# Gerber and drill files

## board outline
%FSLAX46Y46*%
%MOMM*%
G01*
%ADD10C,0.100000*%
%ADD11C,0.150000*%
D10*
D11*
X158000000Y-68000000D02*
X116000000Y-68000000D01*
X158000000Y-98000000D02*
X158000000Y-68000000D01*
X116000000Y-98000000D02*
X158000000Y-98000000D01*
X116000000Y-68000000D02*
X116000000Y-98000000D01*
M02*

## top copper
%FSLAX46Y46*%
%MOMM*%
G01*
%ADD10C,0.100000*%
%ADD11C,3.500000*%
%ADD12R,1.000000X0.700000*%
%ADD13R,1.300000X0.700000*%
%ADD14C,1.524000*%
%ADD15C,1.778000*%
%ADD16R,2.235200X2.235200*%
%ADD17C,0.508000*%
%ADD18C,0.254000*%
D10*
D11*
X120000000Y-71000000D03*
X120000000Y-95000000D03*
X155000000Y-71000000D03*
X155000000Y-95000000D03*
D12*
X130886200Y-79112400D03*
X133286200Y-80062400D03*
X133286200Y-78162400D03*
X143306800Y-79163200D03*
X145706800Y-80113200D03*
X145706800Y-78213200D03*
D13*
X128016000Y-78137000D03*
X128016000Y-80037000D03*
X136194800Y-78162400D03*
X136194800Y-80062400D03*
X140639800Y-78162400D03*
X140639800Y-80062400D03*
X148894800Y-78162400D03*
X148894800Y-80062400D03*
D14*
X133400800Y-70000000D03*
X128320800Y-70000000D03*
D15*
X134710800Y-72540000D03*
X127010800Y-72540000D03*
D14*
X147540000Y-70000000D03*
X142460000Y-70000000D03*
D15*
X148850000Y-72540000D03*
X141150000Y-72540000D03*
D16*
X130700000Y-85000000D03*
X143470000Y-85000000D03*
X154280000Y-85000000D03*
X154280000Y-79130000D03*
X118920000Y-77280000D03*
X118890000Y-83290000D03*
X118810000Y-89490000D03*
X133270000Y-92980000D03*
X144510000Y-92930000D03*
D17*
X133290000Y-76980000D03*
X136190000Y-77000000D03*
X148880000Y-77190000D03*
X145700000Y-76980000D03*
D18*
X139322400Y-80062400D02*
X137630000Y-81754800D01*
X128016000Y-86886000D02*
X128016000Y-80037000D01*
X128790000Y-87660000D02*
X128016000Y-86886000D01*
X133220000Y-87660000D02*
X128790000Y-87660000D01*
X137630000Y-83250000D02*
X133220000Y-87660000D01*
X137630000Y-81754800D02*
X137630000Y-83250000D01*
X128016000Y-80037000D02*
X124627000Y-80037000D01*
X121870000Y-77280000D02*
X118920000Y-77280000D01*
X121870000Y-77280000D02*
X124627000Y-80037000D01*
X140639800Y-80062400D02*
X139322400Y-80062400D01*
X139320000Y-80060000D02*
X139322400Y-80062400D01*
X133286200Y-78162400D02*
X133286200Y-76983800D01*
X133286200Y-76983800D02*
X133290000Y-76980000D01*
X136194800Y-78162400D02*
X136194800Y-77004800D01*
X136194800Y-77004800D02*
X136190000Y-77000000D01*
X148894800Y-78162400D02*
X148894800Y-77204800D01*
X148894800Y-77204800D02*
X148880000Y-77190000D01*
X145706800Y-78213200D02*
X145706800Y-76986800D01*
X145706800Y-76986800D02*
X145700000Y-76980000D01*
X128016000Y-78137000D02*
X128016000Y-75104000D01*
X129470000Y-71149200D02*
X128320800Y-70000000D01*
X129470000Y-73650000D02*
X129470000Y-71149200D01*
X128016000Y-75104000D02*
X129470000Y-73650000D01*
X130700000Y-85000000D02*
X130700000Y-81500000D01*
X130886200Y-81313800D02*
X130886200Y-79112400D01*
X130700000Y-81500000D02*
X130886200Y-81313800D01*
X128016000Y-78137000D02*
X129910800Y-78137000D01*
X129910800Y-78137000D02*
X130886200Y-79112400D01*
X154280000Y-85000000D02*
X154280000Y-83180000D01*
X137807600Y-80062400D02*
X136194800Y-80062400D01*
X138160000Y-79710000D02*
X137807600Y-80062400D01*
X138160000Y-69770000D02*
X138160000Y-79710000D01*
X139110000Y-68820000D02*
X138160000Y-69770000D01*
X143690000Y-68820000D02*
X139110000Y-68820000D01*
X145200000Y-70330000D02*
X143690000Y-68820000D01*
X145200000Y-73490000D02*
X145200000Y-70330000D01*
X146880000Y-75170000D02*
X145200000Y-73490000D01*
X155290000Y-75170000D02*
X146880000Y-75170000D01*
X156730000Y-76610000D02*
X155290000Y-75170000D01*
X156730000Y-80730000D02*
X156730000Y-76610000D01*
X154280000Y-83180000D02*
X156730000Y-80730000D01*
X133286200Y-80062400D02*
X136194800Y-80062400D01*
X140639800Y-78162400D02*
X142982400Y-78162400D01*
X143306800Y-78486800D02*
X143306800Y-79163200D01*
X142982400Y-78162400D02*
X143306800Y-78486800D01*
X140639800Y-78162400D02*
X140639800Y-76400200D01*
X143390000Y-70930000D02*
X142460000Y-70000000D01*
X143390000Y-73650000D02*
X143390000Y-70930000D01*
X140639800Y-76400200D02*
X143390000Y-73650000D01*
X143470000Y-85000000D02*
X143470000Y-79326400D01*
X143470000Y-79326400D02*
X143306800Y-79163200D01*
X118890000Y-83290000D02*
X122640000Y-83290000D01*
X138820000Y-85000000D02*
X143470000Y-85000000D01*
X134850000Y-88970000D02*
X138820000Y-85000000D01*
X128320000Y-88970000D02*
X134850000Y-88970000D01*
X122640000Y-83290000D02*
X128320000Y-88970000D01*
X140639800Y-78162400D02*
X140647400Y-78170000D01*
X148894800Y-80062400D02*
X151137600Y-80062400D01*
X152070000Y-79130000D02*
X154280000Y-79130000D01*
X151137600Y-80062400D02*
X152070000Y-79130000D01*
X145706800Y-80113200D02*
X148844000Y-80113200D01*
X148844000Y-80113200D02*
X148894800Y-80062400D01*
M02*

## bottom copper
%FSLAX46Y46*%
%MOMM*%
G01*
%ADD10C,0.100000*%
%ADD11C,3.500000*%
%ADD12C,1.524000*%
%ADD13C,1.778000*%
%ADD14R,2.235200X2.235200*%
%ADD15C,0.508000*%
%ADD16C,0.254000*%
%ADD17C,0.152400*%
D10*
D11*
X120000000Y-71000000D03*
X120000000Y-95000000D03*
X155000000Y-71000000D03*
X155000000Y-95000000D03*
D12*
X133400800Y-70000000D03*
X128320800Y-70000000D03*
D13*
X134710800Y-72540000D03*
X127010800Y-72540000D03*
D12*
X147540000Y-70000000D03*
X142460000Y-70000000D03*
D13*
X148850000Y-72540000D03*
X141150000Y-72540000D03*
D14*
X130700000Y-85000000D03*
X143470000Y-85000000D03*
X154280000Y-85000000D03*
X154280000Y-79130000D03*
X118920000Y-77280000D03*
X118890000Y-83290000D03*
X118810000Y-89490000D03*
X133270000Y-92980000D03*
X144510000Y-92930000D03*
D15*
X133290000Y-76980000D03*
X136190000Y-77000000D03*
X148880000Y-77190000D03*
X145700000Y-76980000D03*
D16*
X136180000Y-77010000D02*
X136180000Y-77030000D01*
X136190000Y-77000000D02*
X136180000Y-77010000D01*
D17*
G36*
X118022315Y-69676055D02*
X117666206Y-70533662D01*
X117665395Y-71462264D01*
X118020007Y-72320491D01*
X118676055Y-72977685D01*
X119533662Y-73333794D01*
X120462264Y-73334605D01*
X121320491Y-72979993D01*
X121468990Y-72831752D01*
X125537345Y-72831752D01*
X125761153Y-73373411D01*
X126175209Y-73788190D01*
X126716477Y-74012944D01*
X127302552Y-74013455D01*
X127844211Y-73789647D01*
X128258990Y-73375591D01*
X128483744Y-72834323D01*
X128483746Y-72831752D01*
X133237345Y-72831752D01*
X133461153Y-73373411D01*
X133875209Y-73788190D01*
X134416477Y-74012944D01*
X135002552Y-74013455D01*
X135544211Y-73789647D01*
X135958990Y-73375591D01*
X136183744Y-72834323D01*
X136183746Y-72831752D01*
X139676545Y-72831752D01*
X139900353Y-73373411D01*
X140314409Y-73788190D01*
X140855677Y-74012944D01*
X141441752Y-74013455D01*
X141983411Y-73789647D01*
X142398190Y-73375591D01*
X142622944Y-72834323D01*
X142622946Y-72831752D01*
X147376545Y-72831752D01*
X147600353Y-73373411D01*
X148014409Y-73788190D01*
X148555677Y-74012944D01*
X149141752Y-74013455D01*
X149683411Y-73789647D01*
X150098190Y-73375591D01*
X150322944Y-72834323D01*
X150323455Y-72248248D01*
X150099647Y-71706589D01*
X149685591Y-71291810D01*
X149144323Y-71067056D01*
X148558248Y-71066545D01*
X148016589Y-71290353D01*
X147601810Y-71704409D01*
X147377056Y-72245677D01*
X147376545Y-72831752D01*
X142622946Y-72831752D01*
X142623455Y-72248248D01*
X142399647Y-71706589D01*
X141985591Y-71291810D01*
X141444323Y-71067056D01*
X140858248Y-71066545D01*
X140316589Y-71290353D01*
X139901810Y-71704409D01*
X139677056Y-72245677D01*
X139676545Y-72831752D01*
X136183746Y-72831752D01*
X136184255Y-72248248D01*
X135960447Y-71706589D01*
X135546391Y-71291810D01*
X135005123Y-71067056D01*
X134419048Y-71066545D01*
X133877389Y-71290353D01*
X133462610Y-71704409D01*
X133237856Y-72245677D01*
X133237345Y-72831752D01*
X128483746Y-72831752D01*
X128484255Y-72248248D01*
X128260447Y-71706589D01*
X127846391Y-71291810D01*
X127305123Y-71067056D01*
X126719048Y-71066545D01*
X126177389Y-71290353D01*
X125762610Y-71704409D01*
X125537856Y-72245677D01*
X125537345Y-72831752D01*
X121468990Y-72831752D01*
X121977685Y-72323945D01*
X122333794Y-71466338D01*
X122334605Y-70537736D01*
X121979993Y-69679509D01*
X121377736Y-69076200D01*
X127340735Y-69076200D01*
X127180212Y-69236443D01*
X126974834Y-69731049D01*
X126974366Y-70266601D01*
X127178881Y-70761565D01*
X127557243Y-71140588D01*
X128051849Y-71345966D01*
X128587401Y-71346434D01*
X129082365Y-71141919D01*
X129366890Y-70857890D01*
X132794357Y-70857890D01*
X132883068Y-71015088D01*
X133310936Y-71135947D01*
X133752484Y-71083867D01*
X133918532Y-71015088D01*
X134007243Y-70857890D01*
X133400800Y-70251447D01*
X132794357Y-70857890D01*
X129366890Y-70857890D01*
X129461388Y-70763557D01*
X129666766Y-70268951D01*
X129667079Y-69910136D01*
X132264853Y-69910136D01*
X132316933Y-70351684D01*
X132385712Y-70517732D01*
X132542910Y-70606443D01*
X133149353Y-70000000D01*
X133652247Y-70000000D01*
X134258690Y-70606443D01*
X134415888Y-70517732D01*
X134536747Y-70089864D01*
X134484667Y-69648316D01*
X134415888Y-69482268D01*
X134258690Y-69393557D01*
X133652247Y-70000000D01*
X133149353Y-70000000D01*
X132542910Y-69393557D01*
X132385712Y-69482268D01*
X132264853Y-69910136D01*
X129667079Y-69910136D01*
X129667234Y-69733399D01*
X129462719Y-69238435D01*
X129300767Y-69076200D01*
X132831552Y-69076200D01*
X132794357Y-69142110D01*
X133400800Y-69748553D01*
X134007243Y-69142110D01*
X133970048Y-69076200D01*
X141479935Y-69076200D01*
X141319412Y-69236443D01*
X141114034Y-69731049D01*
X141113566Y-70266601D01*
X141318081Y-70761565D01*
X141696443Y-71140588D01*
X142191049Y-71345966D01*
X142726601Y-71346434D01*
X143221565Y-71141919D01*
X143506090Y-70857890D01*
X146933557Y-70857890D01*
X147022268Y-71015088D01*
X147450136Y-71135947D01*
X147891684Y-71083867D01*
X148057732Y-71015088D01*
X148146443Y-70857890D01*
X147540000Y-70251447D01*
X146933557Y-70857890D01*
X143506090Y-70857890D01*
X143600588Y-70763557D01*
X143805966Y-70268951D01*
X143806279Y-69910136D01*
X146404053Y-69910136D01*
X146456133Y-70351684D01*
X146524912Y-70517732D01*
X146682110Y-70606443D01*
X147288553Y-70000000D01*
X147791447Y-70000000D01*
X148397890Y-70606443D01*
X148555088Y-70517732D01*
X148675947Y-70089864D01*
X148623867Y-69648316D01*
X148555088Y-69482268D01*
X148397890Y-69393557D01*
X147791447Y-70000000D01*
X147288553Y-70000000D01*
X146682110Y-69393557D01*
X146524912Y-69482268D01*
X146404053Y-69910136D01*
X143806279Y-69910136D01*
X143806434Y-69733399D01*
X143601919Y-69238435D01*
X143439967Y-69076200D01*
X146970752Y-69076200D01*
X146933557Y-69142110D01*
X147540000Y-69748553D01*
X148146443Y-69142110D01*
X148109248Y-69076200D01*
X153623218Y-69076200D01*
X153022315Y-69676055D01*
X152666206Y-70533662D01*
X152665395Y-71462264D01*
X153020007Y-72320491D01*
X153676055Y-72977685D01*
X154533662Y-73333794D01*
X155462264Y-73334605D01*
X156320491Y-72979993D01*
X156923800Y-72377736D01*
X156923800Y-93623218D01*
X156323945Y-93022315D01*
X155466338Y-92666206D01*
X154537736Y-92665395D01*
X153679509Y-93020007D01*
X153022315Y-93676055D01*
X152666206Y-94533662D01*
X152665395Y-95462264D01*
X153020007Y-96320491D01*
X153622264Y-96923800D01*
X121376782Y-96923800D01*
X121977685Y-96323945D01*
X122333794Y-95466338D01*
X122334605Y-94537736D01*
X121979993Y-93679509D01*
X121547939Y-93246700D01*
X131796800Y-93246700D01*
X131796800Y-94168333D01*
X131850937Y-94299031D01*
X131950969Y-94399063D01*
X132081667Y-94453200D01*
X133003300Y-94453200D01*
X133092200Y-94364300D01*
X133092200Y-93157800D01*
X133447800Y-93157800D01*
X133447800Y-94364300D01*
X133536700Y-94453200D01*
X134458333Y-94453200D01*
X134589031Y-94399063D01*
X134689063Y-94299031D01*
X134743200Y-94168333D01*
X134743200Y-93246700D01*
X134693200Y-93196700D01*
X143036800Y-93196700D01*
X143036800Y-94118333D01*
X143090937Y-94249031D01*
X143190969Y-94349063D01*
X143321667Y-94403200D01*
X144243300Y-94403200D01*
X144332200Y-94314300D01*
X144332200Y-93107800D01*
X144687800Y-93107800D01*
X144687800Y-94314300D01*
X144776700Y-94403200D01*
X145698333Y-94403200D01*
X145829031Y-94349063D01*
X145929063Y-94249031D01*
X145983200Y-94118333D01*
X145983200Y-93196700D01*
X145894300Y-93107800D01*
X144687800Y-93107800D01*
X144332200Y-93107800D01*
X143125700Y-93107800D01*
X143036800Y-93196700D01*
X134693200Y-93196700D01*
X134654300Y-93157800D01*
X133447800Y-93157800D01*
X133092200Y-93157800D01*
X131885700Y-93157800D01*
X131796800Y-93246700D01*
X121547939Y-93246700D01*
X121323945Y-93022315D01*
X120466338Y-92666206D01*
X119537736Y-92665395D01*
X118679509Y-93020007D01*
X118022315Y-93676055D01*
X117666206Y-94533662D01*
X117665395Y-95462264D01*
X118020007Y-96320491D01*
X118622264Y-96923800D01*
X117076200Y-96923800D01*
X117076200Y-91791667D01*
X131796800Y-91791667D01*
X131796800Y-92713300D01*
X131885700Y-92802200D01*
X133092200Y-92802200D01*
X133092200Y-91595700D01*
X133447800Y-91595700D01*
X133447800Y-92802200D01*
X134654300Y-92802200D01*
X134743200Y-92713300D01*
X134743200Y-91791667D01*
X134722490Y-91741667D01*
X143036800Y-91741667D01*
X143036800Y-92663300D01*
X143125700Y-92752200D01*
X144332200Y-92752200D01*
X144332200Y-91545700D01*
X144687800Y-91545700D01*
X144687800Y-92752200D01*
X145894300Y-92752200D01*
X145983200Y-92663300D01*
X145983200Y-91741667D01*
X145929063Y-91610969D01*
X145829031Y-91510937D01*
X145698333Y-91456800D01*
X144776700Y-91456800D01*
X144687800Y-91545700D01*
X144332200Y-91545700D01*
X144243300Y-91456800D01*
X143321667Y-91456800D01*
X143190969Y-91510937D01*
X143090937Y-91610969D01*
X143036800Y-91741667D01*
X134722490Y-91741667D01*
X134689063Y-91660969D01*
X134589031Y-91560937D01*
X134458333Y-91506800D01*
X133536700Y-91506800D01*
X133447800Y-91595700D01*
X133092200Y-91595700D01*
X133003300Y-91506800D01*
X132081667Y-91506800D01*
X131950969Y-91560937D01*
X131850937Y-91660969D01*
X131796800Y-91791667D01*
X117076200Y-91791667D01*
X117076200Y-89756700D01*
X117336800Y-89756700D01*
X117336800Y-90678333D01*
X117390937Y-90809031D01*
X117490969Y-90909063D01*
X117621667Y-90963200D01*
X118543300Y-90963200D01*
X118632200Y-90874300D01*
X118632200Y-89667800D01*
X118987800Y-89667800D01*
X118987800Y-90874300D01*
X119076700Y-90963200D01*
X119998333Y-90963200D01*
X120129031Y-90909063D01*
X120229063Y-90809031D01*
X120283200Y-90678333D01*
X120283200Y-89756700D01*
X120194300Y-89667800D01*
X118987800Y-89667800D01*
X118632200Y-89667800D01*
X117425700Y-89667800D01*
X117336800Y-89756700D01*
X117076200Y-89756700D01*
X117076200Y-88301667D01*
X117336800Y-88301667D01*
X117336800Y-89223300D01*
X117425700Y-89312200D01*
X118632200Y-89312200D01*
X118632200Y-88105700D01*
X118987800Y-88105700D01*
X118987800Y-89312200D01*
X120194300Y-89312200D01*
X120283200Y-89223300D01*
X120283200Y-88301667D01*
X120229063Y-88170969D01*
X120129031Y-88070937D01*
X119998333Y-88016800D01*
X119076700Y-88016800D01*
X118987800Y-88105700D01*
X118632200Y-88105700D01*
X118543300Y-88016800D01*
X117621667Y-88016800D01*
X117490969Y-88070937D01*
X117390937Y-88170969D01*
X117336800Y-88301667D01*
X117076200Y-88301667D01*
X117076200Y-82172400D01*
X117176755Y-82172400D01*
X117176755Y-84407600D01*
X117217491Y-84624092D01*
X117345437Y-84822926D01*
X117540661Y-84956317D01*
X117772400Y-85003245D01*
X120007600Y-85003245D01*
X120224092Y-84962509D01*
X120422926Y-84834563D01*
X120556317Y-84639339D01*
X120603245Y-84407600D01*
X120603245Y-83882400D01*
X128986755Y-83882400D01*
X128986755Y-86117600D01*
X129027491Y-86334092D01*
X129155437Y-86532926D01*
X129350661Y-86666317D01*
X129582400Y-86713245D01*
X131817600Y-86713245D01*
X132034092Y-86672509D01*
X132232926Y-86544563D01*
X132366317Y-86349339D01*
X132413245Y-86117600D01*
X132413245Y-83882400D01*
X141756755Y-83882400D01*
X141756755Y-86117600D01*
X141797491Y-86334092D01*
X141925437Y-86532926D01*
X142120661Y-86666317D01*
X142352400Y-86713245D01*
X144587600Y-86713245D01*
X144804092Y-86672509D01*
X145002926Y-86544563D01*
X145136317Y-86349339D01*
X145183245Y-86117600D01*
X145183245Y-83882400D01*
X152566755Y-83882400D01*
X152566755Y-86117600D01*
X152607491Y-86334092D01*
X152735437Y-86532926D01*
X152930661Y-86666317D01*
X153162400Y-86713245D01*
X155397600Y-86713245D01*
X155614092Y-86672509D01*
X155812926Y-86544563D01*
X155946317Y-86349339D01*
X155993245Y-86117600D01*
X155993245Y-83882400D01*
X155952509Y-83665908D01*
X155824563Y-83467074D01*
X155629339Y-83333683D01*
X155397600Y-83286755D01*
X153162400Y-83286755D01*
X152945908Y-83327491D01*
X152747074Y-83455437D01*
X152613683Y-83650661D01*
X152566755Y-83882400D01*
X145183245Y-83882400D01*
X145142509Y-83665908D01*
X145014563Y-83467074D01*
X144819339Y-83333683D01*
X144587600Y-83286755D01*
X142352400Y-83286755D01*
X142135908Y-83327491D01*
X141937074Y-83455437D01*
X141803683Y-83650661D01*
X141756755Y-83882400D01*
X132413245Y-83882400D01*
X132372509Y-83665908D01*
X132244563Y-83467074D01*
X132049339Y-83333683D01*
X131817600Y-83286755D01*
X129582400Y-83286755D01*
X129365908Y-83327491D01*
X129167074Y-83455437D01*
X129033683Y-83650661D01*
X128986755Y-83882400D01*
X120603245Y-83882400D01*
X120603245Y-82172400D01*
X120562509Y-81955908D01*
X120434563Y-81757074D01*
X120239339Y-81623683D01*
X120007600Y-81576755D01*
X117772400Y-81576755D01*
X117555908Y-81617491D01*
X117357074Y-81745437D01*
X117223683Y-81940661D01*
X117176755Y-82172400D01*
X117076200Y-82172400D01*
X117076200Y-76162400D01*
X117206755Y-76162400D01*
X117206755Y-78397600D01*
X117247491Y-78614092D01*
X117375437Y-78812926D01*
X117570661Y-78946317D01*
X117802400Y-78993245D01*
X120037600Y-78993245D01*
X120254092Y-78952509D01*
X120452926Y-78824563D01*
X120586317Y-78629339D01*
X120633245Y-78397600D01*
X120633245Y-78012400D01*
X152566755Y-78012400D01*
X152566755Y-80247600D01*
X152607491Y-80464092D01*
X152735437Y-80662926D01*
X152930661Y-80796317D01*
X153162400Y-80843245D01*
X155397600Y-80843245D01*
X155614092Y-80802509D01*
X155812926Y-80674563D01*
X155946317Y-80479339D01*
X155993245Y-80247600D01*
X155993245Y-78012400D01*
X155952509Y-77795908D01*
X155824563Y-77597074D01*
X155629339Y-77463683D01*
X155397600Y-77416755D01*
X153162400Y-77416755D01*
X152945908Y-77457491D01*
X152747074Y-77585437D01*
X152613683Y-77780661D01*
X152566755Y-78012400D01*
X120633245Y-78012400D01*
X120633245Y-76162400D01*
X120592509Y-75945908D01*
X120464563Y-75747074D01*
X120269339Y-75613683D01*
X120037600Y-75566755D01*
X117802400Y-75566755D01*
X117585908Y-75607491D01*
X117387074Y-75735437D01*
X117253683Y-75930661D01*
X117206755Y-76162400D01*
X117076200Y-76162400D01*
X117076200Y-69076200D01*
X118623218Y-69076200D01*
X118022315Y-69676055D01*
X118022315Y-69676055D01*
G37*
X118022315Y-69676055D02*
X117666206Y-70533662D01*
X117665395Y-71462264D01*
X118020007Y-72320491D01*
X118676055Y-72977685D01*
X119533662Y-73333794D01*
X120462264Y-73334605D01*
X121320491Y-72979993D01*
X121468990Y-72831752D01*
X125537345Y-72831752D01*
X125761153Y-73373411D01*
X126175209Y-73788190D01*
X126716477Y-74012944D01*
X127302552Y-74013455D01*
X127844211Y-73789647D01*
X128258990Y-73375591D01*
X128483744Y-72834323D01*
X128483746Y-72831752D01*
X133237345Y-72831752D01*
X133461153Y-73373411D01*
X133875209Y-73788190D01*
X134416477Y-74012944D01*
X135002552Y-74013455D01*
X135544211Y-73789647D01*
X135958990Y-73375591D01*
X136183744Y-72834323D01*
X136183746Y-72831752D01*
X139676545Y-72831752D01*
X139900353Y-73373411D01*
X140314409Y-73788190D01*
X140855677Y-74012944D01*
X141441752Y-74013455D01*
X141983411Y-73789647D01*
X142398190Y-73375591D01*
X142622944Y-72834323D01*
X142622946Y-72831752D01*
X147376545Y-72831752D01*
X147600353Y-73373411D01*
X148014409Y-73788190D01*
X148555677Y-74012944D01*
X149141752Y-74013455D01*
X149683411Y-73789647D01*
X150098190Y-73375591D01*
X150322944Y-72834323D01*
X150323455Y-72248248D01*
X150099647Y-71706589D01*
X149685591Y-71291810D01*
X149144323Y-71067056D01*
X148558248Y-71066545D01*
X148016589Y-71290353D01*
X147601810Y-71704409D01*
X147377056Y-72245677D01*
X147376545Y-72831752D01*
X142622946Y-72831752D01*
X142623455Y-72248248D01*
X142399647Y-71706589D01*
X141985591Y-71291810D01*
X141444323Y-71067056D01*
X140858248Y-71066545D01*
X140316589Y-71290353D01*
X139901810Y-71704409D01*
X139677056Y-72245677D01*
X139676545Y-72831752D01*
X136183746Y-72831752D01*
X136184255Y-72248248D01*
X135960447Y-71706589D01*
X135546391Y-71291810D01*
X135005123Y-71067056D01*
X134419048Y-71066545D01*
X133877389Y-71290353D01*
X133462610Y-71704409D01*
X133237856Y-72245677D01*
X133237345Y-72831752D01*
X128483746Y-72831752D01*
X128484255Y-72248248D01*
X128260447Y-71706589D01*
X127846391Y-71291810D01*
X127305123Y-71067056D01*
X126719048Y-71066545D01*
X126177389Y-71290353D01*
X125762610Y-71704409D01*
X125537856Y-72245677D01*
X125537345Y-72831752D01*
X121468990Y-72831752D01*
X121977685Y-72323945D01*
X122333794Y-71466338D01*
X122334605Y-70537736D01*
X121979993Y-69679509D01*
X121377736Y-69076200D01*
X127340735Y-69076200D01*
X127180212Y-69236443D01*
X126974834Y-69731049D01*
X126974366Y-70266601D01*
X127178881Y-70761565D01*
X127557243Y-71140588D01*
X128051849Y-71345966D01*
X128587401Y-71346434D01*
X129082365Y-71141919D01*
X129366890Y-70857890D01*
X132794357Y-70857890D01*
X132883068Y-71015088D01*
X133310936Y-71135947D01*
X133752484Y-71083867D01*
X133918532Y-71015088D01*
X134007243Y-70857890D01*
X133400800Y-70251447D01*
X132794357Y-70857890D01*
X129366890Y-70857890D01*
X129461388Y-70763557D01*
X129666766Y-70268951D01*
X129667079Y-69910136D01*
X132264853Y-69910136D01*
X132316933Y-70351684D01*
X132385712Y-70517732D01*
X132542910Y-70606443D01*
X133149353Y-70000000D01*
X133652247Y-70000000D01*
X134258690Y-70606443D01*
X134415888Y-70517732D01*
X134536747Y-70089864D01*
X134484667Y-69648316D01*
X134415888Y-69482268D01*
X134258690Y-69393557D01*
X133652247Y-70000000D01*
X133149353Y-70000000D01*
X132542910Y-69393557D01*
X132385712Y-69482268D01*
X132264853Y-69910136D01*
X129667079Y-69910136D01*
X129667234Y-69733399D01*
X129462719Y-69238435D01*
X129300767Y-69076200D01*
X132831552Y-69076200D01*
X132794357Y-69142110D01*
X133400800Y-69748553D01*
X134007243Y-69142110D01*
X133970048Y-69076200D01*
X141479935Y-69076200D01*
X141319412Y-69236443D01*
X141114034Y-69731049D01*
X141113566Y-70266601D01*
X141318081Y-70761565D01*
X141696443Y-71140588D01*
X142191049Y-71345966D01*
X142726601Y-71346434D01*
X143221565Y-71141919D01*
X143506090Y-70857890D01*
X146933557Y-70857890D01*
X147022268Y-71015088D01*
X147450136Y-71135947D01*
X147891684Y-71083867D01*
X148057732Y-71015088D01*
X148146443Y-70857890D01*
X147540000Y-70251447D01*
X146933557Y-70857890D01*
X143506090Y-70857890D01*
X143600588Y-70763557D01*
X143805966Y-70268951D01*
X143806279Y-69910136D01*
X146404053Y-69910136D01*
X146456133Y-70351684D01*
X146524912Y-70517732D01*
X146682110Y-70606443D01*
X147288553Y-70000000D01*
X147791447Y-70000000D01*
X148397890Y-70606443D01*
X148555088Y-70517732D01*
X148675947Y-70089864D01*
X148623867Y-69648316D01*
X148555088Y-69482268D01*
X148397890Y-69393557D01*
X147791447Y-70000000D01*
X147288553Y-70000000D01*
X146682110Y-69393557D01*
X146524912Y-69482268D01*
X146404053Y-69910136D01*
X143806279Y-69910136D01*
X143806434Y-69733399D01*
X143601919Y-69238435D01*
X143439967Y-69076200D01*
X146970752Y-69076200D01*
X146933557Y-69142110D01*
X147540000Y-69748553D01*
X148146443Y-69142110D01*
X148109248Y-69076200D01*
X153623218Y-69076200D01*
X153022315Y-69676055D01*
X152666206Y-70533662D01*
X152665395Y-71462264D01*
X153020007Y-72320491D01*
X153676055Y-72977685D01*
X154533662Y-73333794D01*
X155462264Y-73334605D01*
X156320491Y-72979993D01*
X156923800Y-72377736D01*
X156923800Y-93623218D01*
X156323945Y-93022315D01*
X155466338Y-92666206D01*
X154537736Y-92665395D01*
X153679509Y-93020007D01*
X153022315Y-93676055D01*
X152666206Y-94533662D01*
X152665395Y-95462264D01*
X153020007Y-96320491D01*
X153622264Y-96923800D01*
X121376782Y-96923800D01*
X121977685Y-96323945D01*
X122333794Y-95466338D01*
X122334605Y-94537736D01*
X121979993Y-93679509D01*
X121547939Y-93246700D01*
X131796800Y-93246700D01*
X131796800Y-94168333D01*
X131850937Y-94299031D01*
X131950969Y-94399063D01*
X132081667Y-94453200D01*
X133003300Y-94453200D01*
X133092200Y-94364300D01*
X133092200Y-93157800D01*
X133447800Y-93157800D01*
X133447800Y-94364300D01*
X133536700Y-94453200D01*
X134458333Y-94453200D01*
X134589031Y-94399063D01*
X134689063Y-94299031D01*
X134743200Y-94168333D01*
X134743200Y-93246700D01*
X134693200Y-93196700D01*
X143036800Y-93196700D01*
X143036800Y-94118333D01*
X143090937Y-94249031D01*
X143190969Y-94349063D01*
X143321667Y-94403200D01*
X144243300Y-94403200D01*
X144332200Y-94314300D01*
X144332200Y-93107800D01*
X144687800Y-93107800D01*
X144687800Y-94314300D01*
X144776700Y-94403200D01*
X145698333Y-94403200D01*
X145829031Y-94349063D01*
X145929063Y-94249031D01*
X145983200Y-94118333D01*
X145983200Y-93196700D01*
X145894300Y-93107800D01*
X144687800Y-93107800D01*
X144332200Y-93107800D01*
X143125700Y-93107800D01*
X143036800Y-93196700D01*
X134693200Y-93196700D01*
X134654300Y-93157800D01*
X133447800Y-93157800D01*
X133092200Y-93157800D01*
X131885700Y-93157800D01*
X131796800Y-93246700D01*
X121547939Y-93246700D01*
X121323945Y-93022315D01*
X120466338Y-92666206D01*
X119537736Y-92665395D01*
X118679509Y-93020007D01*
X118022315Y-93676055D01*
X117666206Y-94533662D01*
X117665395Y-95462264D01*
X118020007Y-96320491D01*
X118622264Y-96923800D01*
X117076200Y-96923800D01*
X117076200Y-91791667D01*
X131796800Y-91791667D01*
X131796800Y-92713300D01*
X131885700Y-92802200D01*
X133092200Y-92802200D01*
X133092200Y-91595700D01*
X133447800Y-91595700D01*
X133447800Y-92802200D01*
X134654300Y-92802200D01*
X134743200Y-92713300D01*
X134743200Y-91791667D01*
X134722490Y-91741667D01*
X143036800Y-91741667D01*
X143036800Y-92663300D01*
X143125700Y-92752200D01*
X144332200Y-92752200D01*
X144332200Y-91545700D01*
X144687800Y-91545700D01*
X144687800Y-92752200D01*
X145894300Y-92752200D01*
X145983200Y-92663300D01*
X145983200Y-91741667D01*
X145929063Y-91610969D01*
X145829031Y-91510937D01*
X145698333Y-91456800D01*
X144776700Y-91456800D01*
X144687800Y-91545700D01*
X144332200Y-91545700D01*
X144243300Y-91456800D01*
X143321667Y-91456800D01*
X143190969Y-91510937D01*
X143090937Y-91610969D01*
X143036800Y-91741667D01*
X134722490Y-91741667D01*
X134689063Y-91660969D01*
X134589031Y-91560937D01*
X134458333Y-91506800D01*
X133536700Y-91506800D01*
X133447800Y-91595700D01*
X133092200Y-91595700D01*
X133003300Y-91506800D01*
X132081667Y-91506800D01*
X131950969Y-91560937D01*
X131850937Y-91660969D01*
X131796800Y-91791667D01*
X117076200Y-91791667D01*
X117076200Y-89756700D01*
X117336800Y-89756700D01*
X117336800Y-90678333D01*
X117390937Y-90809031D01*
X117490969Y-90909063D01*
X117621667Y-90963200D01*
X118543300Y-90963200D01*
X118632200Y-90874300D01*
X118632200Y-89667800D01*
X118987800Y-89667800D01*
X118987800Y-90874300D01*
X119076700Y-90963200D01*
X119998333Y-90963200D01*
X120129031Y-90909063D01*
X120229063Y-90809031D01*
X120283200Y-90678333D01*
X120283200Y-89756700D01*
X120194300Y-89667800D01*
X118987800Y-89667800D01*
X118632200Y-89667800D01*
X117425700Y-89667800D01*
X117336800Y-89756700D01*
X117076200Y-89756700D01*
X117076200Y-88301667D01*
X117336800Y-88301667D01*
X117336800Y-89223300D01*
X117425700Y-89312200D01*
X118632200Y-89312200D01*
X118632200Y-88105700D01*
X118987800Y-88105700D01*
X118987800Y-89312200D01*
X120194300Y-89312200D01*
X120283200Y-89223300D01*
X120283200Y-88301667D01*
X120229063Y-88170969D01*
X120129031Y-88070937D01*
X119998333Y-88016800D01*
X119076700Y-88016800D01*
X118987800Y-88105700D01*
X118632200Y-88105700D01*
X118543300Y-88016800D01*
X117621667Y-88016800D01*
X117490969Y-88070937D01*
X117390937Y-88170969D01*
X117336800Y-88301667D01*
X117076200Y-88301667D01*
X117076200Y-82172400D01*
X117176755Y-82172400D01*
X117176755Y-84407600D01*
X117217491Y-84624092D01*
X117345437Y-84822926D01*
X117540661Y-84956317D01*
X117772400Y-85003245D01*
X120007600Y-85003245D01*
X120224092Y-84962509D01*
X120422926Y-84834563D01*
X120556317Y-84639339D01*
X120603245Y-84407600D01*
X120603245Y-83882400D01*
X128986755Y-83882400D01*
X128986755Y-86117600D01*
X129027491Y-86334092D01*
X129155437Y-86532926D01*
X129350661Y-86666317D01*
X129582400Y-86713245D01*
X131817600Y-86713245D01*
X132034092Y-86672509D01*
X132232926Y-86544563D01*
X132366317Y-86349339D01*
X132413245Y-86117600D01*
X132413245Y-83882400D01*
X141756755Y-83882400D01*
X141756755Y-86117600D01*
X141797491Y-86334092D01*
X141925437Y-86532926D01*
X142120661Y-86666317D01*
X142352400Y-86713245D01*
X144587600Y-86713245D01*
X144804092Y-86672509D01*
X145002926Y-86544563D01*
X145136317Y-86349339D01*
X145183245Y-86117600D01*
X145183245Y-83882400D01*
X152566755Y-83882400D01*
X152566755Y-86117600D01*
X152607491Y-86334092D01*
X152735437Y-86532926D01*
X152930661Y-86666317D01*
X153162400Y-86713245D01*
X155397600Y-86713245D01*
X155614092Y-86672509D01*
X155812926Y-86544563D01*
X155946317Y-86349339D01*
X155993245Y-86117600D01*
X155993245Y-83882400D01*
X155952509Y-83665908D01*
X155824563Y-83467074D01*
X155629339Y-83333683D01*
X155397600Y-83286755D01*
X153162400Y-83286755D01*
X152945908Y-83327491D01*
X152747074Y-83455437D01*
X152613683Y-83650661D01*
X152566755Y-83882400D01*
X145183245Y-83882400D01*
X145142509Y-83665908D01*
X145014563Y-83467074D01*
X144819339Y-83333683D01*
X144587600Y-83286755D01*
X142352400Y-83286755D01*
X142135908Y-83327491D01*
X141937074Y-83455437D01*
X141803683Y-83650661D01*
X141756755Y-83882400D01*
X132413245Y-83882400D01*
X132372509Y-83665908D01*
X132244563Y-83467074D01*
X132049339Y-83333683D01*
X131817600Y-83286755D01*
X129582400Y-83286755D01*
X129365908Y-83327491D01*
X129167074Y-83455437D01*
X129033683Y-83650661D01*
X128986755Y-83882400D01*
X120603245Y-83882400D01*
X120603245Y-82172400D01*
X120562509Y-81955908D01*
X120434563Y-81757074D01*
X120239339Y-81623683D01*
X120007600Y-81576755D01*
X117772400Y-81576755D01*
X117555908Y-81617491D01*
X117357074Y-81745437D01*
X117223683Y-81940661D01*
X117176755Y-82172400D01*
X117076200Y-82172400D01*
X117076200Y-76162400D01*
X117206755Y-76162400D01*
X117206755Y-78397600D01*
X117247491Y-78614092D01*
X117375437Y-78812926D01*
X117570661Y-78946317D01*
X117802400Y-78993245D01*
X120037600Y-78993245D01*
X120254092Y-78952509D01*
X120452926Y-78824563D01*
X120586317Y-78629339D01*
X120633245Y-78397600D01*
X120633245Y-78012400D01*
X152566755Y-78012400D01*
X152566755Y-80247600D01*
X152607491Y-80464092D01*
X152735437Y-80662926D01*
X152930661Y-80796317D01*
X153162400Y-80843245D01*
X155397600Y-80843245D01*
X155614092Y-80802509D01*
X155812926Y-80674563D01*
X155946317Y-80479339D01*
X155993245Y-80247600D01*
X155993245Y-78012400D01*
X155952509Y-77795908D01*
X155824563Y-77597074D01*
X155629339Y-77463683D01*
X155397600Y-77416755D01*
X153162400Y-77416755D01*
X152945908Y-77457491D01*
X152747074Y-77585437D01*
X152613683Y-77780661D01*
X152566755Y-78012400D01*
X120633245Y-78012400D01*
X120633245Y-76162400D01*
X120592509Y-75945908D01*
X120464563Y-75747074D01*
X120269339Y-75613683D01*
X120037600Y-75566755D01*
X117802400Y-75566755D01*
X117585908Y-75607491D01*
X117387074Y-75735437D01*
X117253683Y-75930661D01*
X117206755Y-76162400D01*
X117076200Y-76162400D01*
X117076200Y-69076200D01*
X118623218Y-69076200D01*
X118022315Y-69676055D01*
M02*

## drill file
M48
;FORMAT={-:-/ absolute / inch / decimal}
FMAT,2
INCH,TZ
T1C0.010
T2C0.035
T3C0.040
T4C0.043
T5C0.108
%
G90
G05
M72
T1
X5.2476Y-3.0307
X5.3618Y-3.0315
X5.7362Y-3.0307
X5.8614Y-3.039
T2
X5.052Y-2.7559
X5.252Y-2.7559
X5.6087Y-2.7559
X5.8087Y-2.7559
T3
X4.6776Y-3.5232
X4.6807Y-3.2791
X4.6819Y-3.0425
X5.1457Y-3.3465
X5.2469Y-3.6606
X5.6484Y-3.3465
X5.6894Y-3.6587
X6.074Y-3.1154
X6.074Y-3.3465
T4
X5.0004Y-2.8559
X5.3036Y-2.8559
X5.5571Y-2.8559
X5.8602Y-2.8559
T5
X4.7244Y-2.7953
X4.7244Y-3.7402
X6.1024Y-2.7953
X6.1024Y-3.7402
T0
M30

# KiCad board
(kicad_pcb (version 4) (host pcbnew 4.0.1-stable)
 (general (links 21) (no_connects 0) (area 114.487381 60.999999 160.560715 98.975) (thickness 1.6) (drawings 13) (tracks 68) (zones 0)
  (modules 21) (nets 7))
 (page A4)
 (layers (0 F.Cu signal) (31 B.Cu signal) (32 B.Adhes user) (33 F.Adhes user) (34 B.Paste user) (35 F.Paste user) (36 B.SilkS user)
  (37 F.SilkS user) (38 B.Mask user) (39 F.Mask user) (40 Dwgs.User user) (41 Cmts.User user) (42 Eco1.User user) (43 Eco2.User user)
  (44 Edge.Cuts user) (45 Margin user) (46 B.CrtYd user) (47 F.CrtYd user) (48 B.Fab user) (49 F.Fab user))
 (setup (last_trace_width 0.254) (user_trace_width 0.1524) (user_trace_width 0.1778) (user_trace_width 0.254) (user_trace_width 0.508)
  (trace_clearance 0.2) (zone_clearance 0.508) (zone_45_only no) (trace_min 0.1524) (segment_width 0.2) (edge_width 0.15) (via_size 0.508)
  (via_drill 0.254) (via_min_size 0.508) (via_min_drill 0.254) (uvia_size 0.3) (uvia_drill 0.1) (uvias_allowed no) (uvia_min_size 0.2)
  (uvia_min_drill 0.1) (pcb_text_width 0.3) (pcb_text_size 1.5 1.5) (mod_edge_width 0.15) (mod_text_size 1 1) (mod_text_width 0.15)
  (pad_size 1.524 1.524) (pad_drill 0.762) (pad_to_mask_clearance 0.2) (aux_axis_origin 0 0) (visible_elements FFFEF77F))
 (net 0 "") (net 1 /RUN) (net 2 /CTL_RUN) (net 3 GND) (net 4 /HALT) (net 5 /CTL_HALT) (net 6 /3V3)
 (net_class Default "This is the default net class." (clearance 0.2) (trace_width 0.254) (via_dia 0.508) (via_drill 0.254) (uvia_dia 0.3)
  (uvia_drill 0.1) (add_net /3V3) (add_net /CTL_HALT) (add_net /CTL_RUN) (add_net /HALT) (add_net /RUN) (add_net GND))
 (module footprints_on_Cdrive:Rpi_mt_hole (layer F.Cu) (at 120 71)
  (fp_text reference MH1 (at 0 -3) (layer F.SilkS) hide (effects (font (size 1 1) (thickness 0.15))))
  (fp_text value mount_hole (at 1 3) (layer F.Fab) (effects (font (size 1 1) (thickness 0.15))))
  (pad 0 thru_hole circle (at 0 0) (size 3.5 3.5) (drill 2.75) (layers *.Cu *.Mask F.SilkS)))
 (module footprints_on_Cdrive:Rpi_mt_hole (layer F.Cu) (at 120 95)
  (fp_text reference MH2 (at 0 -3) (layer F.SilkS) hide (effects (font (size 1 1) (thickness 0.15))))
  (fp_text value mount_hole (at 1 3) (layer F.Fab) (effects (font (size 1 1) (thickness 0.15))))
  (pad 0 thru_hole circle (at 0 0) (size 3.5 3.5) (drill 2.75) (layers *.Cu *.Mask F.SilkS)))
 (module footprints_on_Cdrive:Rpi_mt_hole (layer F.Cu) (at 155 71)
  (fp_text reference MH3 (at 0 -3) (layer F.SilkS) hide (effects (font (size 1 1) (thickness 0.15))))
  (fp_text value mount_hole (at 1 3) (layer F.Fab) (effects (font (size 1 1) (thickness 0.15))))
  (pad 0 thru_hole circle (at 0 0) (size 3.5 3.5) (drill 2.75) (layers *.Cu *.Mask F.SilkS)))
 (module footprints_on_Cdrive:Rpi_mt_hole (layer F.Cu) (at 155 95)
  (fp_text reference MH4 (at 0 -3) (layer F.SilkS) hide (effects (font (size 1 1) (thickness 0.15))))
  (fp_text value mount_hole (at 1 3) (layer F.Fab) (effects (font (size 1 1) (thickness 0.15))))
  (pad 0 thru_hole circle (at 0 0) (size 3.5 3.5) (drill 2.75) (layers *.Cu *.Mask F.SilkS)))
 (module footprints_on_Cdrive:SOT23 (layer F.Cu) (at 130.8862 79.1124 90)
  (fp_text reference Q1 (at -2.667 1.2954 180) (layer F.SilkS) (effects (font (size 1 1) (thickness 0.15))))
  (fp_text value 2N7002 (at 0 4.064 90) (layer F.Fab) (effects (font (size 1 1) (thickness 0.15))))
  (pad 3 smd rect (at 0 0 90) (size 0.7 1) (layers F.Cu F.Paste F.Mask) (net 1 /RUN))
  (pad 1 smd rect (at -0.95 2.4 90) (size 0.7 1) (layers F.Cu F.Paste F.Mask) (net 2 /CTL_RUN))
  (pad 2 smd rect (at 0.95 2.4 90) (size 0.7 1) (layers F.Cu F.Paste F.Mask) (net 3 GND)))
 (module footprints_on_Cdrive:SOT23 (layer F.Cu) (at 143.3068 79.1632 90)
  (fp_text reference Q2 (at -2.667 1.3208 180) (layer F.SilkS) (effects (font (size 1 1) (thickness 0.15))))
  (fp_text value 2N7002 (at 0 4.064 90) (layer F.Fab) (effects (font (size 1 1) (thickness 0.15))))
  (pad 3 smd rect (at 0 0 90) (size 0.7 1) (layers F.Cu F.Paste F.Mask) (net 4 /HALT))
  (pad 1 smd rect (at -0.95 2.4 90) (size 0.7 1) (layers F.Cu F.Paste F.Mask) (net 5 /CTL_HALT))
  (pad 2 smd rect (at 0.95 2.4 90) (size 0.7 1) (layers F.Cu F.Paste F.Mask) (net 3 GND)))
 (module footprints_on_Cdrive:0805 (layer F.Cu) (at 128.016 79.087 270)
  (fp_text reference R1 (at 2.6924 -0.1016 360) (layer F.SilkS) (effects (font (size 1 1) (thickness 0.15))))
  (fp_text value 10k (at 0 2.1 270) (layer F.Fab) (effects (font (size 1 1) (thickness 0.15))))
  (pad 1 smd rect (at -0.95 0 270) (size 0.7 1.3) (layers F.Cu F.Paste F.Mask) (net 1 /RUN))
  (pad 2 smd rect (at 0.95 0 270) (size 0.7 1.3) (layers F.Cu F.Paste F.Mask) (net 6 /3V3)))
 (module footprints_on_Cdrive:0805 (layer F.Cu) (at 136.1948 79.1124 270)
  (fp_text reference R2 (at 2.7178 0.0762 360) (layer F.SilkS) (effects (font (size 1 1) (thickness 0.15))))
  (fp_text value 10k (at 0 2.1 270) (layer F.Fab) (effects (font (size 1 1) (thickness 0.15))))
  (pad 1 smd rect (at -0.95 0 270) (size 0.7 1.3) (layers F.Cu F.Paste F.Mask) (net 3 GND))
  (pad 2 smd rect (at 0.95 0 270) (size 0.7 1.3) (layers F.Cu F.Paste F.Mask) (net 2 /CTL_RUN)))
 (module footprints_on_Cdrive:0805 (layer F.Cu) (at 140.6398 79.1124 270)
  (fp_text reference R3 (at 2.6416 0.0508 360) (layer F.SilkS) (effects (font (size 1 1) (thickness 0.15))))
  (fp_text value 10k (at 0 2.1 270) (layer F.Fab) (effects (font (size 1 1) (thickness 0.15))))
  (pad 1 smd rect (at -0.95 0 270) (size 0.7 1.3) (layers F.Cu F.Paste F.Mask) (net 4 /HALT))
  (pad 2 smd rect (at 0.95 0 270) (size 0.7 1.3) (layers F.Cu F.Paste F.Mask) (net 6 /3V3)))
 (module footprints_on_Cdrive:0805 (layer F.Cu) (at 148.8948 79.1124 270)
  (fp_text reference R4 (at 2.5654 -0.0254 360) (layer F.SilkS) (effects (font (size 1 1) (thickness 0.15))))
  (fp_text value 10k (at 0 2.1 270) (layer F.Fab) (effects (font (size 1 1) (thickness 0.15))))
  (pad 1 smd rect (at -0.95 0 270) (size 0.7 1.3) (layers F.Cu F.Paste F.Mask) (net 3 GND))
  (pad 2 smd rect (at 0.95 0 270) (size 0.7 1.3) (layers F.Cu F.Paste F.Mask) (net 5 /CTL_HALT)))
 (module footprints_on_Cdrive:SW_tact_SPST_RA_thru (layer F.Cu) (at 130.8608 70 180)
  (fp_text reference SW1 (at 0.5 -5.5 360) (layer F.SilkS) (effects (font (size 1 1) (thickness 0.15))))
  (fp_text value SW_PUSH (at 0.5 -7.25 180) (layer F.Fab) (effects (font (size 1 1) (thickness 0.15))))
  (pad 1 thru_hole circle (at -2.54 0 180) (size 1.524 1.524) (drill 0.889) (layers *.Cu *.Mask F.SilkS) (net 3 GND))
  (pad 2 thru_hole circle (at 2.54 0 180) (size 1.524 1.524) (drill 0.889) (layers *.Cu *.Mask F.SilkS) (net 1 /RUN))
  (pad 0 thru_hole circle (at -3.85 -2.54 180) (size 1.778 1.778) (drill 1.0922) (layers *.Cu *.Mask F.SilkS))
  (pad 0 thru_hole circle (at 3.85 -2.54 180) (size 1.778 1.778) (drill 1.0922) (layers *.Cu *.Mask F.SilkS)))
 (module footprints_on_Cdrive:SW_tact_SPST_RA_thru (layer F.Cu) (at 145 70 180)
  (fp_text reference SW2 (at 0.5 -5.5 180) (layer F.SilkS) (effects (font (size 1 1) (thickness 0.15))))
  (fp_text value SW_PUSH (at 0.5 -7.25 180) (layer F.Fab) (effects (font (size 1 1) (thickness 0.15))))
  (pad 1 thru_hole circle (at -2.54 0 180) (size 1.524 1.524) (drill 0.889) (layers *.Cu *.Mask F.SilkS) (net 3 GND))
  (pad 2 thru_hole circle (at 2.54 0 180) (size 1.524 1.524) (drill 0.889) (layers *.Cu *.Mask F.SilkS) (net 4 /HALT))
  (pad 0 thru_hole circle (at -3.85 -2.54 180) (size 1.778 1.778) (drill 1.0922) (layers *.Cu *.Mask F.SilkS))
  (pad 0 thru_hole circle (at 3.85 -2.54 180) (size 1.778 1.778) (drill 1.0922) (layers *.Cu *.Mask F.SilkS)))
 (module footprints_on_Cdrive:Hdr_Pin (layer F.Cu) (at 130.7 85)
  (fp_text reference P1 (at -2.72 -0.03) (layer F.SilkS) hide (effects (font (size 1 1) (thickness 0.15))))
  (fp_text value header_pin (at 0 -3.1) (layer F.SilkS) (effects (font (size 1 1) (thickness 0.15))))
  (pad 1 thru_hole rect (at 0 0) (size 2.2352 2.2352) (drill 1.016) (layers *.Cu *.Mask F.SilkS) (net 1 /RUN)))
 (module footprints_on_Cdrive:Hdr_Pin (layer F.Cu) (at 143.47 85)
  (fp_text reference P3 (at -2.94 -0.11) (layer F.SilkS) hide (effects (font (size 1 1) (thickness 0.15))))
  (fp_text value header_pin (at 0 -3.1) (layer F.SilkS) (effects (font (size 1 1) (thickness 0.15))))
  (pad 1 thru_hole rect (at 0 0) (size 2.2352 2.2352) (drill 1.016) (layers *.Cu *.Mask F.SilkS) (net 4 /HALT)))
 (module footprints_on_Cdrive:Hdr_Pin (layer F.Cu) (at 154.28 85)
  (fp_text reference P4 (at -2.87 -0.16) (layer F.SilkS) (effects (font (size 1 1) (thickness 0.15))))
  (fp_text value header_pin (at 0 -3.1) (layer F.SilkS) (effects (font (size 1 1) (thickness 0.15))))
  (pad 1 thru_hole rect (at 0 0) (size 2.2352 2.2352) (drill 1.016) (layers *.Cu *.Mask F.SilkS) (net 2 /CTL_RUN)))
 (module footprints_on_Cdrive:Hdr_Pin (layer F.Cu) (at 154.28 79.13)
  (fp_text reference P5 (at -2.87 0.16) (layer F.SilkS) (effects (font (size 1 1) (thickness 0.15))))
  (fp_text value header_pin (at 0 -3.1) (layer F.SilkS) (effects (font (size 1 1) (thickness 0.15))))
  (pad 1 thru_hole rect (at 0 0) (size 2.2352 2.2352) (drill 1.016) (layers *.Cu *.Mask F.SilkS) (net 5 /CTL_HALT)))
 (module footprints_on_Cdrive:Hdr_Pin (layer F.Cu) (at 118.92 77.28)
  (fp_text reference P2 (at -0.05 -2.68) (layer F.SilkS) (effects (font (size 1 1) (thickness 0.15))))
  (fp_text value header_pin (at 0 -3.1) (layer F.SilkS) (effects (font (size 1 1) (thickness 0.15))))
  (pad 1 thru_hole rect (at 0 0) (size 2.2352 2.2352) (drill 1.016) (layers *.Cu *.Mask F.SilkS) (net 6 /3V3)))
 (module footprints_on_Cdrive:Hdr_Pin (layer F.Cu) (at 118.89 83.29)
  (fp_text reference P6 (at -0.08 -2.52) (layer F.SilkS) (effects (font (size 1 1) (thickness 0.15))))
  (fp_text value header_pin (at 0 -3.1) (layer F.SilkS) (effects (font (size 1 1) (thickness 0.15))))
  (pad 1 thru_hole rect (at 0 0) (size 2.2352 2.2352) (drill 1.016) (layers *.Cu *.Mask F.SilkS) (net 4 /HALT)))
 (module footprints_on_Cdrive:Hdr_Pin (layer F.Cu) (at 118.81 89.49)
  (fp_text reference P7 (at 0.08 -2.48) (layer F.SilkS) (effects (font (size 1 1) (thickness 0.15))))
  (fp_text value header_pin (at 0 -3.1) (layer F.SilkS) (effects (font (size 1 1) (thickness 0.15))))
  (pad 1 thru_hole rect (at 0 0) (size 2.2352 2.2352) (drill 1.016) (layers *.Cu *.Mask F.SilkS) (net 3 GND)))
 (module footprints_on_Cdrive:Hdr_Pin (layer F.Cu) (at 133.27 92.98)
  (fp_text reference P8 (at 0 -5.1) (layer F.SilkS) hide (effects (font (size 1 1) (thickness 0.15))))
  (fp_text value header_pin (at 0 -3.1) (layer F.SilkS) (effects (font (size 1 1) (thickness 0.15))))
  (pad 1 thru_hole rect (at 0 0) (size 2.2352 2.2352) (drill 1.016) (layers *.Cu *.Mask F.SilkS) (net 3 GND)))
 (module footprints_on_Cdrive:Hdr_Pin (layer F.Cu) (at 144.51 92.93)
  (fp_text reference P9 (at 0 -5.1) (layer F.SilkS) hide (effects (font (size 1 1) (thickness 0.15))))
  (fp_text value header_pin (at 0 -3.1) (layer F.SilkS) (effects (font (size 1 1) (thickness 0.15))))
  (pad 1 thru_hole rect (at 0 0) (size 2.2352 2.2352) (drill 1.016) (layers *.Cu *.Mask F.SilkS) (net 3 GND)))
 (gr_line (start 158 68) (end 116 68) (angle 90) (layer Edge.Cuts) (width 0.15))
 (gr_line (start 158 98) (end 158 68) (angle 90) (layer Edge.Cuts) (width 0.15))
 (gr_line (start 116 98) (end 158 98) (angle 90) (layer Edge.Cuts) (width 0.15))
 (gr_line (start 116 68) (end 116 98) (angle 90) (layer Edge.Cuts) (width 0.15))
 (segment (start 139.3224 80.0624) (end 137.63 81.7548) (width 0.254) (layer F.Cu) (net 6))
 (segment (start 128.016 86.886) (end 128.016 80.037) (width 0.254) (layer F.Cu) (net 6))
 (segment (start 128.79 87.66) (end 128.016 86.886) (width 0.254) (layer F.Cu) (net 6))
 (segment (start 133.22 87.66) (end 128.79 87.66) (width 0.254) (layer F.Cu) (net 6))
 (segment (start 137.63 83.25) (end 133.22 87.66) (width 0.254) (layer F.Cu) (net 6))
 (segment (start 137.63 81.7548) (end 137.63 83.25) (width 0.254) (layer F.Cu) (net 6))
 (segment (start 128.016 80.037) (end 124.627 80.037) (width 0.254) (layer F.Cu) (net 6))
 (segment (start 121.87 77.28) (end 118.92 77.28) (width 0.254) (layer F.Cu) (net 6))
 (segment (start 121.87 77.28) (end 124.627 80.037) (width 0.254) (layer F.Cu) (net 6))
 (segment (start 140.6398 80.0624) (end 139.3224 80.0624) (width 0.254) (layer F.Cu) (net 6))
 (segment (start 139.32 80.06) (end 139.3224 80.0624) (width 0.254) (layer F.Cu) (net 6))
 (segment (start 133.2862 78.1624) (end 133.2862 76.9838) (width 0.254) (layer F.Cu) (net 3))
 (via (at 133.29 76.98) (size 0.508) (drill 0.254) (layers F.Cu B.Cu) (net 3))
 (segment (start 133.2862 76.9838) (end 133.29 76.98) (width 0.254) (layer F.Cu) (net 3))
 (segment (start 136.1948 78.1624) (end 136.1948 77.0048) (width 0.254) (layer F.Cu) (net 3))
 (segment (start 136.18 77.01) (end 136.18 77.03) (width 0.254) (layer B.Cu) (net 3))
 (segment (start 136.19 77) (end 136.18 77.01) (width 0.254) (layer B.Cu) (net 3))
 (via (at 136.19 77) (size 0.508) (drill 0.254) (layers F.Cu B.Cu) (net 3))
 (segment (start 136.1948 77.0048) (end 136.19 77) (width 0.254) (layer F.Cu) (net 3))
 (segment (start 148.8948 78.1624) (end 148.8948 77.2048) (width 0.254) (layer F.Cu) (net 3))
 (via (at 148.88 77.19) (size 0.508) (drill 0.254) (layers F.Cu B.Cu) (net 3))
 (segment (start 148.8948 77.2048) (end 148.88 77.19) (width 0.254) (layer F.Cu) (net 3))
 (segment (start 145.7068 78.2132) (end 145.7068 76.9868) (width 0.254) (layer F.Cu) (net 3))
 (via (at 145.7 76.98) (size 0.508) (drill 0.254) (layers F.Cu B.Cu) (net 3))
 (segment (start 145.7068 76.9868) (end 145.7 76.98) (width 0.254) (layer F.Cu) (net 3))
 (segment (start 128.016 78.137) (end 128.016 75.104) (width 0.254) (layer F.Cu) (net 1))
 (segment (start 129.47 71.1492) (end 128.3208 70) (width 0.254) (layer F.Cu) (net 1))
 (segment (start 129.47 73.65) (end 129.47 71.1492) (width 0.254) (layer F.Cu) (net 1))
 (segment (start 128.016 75.104) (end 129.47 73.65) (width 0.254) (layer F.Cu) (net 1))
 (segment (start 130.7 85) (end 130.7 81.5) (width 0.254) (layer F.Cu) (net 1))
 (segment (start 130.8862 81.3138) (end 130.8862 79.1124) (width 0.254) (layer F.Cu) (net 1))
 (segment (start 130.7 81.5) (end 130.8862 81.3138) (width 0.254) (layer F.Cu) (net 1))
 (segment (start 128.016 78.137) (end 129.9108 78.137) (width 0.254) (layer F.Cu) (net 1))
 (segment (start 129.9108 78.137) (end 130.8862 79.1124) (width 0.254) (layer F.Cu) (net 1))
 (segment (start 154.28 85) (end 154.28 83.18) (width 0.254) (layer F.Cu) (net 2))
 (segment (start 137.8076 80.0624) (end 136.1948 80.0624) (width 0.254) (layer F.Cu) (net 2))
 (segment (start 138.16 79.71) (end 137.8076 80.0624) (width 0.254) (layer F.Cu) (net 2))
 (segment (start 138.16 69.77) (end 138.16 79.71) (width 0.254) (layer F.Cu) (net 2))
 (segment (start 139.11 68.82) (end 138.16 69.77) (width 0.254) (layer F.Cu) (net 2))
 (segment (start 143.69 68.82) (end 139.11 68.82) (width 0.254) (layer F.Cu) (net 2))
 (segment (start 145.2 70.33) (end 143.69 68.82) (width 0.254) (layer F.Cu) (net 2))
 (segment (start 145.2 73.49) (end 145.2 70.33) (width 0.254) (layer F.Cu) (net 2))
 (segment (start 146.88 75.17) (end 145.2 73.49) (width 0.254) (layer F.Cu) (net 2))
 (segment (start 155.29 75.17) (end 146.88 75.17) (width 0.254) (layer F.Cu) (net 2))
 (segment (start 156.73 76.61) (end 155.29 75.17) (width 0.254) (layer F.Cu) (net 2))
 (segment (start 156.73 80.73) (end 156.73 76.61) (width 0.254) (layer F.Cu) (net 2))
 (segment (start 154.28 83.18) (end 156.73 80.73) (width 0.254) (layer F.Cu) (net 2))
 (segment (start 133.2862 80.0624) (end 136.1948 80.0624) (width 0.254) (layer F.Cu) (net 2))
 (segment (start 140.6398 78.1624) (end 142.9824 78.1624) (width 0.254) (layer F.Cu) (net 4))
 (segment (start 143.3068 78.4868) (end 143.3068 79.1632) (width 0.254) (layer F.Cu) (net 4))
 (segment (start 142.9824 78.1624) (end 143.3068 78.4868) (width 0.254) (layer F.Cu) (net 4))
 (segment (start 140.6398 78.1624) (end 140.6398 76.4002) (width 0.254) (layer F.Cu) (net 4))
 (segment (start 143.39 70.93) (end 142.46 70) (width 0.254) (layer F.Cu) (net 4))
 (segment (start 143.39 73.65) (end 143.39 70.93) (width 0.254) (layer F.Cu) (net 4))
 (segment (start 140.6398 76.4002) (end 143.39 73.65) (width 0.254) (layer F.Cu) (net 4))
 (segment (start 143.47 85) (end 143.47 79.3264) (width 0.254) (layer F.Cu) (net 4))
 (segment (start 143.47 79.3264) (end 143.3068 79.1632) (width 0.254) (layer F.Cu) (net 4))
 (segment (start 118.89 83.29) (end 122.64 83.29) (width 0.254) (layer F.Cu) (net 4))
 (segment (start 138.82 85) (end 143.47 85) (width 0.254) (layer F.Cu) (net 4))
 (segment (start 134.85 88.97) (end 138.82 85) (width 0.254) (layer F.Cu) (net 4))
 (segment (start 128.32 88.97) (end 134.85 88.97) (width 0.254) (layer F.Cu) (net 4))
 (segment (start 122.64 83.29) (end 128.32 88.97) (width 0.254) (layer F.Cu) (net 4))
 (segment (start 140.6398 78.1624) (end 140.6474 78.17) (width 0.254) (layer F.Cu) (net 4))
 (segment (start 148.8948 80.0624) (end 151.1376 80.0624) (width 0.254) (layer F.Cu) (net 5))
 (segment (start 152.07 79.13) (end 154.28 79.13) (width 0.254) (layer F.Cu) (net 5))
 (segment (start 151.1376 80.0624) (end 152.07 79.13) (width 0.254) (layer F.Cu) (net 5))
 (segment (start 145.7068 80.1132) (end 148.844 80.1132) (width 0.254) (layer F.Cu) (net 5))
 (segment (start 148.844 80.1132) (end 148.8948 80.0624) (width 0.254) (layer F.Cu) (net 5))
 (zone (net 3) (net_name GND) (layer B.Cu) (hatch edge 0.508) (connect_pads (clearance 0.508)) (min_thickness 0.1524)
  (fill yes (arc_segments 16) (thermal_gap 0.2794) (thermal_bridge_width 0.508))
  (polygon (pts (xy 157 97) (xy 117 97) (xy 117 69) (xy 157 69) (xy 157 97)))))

